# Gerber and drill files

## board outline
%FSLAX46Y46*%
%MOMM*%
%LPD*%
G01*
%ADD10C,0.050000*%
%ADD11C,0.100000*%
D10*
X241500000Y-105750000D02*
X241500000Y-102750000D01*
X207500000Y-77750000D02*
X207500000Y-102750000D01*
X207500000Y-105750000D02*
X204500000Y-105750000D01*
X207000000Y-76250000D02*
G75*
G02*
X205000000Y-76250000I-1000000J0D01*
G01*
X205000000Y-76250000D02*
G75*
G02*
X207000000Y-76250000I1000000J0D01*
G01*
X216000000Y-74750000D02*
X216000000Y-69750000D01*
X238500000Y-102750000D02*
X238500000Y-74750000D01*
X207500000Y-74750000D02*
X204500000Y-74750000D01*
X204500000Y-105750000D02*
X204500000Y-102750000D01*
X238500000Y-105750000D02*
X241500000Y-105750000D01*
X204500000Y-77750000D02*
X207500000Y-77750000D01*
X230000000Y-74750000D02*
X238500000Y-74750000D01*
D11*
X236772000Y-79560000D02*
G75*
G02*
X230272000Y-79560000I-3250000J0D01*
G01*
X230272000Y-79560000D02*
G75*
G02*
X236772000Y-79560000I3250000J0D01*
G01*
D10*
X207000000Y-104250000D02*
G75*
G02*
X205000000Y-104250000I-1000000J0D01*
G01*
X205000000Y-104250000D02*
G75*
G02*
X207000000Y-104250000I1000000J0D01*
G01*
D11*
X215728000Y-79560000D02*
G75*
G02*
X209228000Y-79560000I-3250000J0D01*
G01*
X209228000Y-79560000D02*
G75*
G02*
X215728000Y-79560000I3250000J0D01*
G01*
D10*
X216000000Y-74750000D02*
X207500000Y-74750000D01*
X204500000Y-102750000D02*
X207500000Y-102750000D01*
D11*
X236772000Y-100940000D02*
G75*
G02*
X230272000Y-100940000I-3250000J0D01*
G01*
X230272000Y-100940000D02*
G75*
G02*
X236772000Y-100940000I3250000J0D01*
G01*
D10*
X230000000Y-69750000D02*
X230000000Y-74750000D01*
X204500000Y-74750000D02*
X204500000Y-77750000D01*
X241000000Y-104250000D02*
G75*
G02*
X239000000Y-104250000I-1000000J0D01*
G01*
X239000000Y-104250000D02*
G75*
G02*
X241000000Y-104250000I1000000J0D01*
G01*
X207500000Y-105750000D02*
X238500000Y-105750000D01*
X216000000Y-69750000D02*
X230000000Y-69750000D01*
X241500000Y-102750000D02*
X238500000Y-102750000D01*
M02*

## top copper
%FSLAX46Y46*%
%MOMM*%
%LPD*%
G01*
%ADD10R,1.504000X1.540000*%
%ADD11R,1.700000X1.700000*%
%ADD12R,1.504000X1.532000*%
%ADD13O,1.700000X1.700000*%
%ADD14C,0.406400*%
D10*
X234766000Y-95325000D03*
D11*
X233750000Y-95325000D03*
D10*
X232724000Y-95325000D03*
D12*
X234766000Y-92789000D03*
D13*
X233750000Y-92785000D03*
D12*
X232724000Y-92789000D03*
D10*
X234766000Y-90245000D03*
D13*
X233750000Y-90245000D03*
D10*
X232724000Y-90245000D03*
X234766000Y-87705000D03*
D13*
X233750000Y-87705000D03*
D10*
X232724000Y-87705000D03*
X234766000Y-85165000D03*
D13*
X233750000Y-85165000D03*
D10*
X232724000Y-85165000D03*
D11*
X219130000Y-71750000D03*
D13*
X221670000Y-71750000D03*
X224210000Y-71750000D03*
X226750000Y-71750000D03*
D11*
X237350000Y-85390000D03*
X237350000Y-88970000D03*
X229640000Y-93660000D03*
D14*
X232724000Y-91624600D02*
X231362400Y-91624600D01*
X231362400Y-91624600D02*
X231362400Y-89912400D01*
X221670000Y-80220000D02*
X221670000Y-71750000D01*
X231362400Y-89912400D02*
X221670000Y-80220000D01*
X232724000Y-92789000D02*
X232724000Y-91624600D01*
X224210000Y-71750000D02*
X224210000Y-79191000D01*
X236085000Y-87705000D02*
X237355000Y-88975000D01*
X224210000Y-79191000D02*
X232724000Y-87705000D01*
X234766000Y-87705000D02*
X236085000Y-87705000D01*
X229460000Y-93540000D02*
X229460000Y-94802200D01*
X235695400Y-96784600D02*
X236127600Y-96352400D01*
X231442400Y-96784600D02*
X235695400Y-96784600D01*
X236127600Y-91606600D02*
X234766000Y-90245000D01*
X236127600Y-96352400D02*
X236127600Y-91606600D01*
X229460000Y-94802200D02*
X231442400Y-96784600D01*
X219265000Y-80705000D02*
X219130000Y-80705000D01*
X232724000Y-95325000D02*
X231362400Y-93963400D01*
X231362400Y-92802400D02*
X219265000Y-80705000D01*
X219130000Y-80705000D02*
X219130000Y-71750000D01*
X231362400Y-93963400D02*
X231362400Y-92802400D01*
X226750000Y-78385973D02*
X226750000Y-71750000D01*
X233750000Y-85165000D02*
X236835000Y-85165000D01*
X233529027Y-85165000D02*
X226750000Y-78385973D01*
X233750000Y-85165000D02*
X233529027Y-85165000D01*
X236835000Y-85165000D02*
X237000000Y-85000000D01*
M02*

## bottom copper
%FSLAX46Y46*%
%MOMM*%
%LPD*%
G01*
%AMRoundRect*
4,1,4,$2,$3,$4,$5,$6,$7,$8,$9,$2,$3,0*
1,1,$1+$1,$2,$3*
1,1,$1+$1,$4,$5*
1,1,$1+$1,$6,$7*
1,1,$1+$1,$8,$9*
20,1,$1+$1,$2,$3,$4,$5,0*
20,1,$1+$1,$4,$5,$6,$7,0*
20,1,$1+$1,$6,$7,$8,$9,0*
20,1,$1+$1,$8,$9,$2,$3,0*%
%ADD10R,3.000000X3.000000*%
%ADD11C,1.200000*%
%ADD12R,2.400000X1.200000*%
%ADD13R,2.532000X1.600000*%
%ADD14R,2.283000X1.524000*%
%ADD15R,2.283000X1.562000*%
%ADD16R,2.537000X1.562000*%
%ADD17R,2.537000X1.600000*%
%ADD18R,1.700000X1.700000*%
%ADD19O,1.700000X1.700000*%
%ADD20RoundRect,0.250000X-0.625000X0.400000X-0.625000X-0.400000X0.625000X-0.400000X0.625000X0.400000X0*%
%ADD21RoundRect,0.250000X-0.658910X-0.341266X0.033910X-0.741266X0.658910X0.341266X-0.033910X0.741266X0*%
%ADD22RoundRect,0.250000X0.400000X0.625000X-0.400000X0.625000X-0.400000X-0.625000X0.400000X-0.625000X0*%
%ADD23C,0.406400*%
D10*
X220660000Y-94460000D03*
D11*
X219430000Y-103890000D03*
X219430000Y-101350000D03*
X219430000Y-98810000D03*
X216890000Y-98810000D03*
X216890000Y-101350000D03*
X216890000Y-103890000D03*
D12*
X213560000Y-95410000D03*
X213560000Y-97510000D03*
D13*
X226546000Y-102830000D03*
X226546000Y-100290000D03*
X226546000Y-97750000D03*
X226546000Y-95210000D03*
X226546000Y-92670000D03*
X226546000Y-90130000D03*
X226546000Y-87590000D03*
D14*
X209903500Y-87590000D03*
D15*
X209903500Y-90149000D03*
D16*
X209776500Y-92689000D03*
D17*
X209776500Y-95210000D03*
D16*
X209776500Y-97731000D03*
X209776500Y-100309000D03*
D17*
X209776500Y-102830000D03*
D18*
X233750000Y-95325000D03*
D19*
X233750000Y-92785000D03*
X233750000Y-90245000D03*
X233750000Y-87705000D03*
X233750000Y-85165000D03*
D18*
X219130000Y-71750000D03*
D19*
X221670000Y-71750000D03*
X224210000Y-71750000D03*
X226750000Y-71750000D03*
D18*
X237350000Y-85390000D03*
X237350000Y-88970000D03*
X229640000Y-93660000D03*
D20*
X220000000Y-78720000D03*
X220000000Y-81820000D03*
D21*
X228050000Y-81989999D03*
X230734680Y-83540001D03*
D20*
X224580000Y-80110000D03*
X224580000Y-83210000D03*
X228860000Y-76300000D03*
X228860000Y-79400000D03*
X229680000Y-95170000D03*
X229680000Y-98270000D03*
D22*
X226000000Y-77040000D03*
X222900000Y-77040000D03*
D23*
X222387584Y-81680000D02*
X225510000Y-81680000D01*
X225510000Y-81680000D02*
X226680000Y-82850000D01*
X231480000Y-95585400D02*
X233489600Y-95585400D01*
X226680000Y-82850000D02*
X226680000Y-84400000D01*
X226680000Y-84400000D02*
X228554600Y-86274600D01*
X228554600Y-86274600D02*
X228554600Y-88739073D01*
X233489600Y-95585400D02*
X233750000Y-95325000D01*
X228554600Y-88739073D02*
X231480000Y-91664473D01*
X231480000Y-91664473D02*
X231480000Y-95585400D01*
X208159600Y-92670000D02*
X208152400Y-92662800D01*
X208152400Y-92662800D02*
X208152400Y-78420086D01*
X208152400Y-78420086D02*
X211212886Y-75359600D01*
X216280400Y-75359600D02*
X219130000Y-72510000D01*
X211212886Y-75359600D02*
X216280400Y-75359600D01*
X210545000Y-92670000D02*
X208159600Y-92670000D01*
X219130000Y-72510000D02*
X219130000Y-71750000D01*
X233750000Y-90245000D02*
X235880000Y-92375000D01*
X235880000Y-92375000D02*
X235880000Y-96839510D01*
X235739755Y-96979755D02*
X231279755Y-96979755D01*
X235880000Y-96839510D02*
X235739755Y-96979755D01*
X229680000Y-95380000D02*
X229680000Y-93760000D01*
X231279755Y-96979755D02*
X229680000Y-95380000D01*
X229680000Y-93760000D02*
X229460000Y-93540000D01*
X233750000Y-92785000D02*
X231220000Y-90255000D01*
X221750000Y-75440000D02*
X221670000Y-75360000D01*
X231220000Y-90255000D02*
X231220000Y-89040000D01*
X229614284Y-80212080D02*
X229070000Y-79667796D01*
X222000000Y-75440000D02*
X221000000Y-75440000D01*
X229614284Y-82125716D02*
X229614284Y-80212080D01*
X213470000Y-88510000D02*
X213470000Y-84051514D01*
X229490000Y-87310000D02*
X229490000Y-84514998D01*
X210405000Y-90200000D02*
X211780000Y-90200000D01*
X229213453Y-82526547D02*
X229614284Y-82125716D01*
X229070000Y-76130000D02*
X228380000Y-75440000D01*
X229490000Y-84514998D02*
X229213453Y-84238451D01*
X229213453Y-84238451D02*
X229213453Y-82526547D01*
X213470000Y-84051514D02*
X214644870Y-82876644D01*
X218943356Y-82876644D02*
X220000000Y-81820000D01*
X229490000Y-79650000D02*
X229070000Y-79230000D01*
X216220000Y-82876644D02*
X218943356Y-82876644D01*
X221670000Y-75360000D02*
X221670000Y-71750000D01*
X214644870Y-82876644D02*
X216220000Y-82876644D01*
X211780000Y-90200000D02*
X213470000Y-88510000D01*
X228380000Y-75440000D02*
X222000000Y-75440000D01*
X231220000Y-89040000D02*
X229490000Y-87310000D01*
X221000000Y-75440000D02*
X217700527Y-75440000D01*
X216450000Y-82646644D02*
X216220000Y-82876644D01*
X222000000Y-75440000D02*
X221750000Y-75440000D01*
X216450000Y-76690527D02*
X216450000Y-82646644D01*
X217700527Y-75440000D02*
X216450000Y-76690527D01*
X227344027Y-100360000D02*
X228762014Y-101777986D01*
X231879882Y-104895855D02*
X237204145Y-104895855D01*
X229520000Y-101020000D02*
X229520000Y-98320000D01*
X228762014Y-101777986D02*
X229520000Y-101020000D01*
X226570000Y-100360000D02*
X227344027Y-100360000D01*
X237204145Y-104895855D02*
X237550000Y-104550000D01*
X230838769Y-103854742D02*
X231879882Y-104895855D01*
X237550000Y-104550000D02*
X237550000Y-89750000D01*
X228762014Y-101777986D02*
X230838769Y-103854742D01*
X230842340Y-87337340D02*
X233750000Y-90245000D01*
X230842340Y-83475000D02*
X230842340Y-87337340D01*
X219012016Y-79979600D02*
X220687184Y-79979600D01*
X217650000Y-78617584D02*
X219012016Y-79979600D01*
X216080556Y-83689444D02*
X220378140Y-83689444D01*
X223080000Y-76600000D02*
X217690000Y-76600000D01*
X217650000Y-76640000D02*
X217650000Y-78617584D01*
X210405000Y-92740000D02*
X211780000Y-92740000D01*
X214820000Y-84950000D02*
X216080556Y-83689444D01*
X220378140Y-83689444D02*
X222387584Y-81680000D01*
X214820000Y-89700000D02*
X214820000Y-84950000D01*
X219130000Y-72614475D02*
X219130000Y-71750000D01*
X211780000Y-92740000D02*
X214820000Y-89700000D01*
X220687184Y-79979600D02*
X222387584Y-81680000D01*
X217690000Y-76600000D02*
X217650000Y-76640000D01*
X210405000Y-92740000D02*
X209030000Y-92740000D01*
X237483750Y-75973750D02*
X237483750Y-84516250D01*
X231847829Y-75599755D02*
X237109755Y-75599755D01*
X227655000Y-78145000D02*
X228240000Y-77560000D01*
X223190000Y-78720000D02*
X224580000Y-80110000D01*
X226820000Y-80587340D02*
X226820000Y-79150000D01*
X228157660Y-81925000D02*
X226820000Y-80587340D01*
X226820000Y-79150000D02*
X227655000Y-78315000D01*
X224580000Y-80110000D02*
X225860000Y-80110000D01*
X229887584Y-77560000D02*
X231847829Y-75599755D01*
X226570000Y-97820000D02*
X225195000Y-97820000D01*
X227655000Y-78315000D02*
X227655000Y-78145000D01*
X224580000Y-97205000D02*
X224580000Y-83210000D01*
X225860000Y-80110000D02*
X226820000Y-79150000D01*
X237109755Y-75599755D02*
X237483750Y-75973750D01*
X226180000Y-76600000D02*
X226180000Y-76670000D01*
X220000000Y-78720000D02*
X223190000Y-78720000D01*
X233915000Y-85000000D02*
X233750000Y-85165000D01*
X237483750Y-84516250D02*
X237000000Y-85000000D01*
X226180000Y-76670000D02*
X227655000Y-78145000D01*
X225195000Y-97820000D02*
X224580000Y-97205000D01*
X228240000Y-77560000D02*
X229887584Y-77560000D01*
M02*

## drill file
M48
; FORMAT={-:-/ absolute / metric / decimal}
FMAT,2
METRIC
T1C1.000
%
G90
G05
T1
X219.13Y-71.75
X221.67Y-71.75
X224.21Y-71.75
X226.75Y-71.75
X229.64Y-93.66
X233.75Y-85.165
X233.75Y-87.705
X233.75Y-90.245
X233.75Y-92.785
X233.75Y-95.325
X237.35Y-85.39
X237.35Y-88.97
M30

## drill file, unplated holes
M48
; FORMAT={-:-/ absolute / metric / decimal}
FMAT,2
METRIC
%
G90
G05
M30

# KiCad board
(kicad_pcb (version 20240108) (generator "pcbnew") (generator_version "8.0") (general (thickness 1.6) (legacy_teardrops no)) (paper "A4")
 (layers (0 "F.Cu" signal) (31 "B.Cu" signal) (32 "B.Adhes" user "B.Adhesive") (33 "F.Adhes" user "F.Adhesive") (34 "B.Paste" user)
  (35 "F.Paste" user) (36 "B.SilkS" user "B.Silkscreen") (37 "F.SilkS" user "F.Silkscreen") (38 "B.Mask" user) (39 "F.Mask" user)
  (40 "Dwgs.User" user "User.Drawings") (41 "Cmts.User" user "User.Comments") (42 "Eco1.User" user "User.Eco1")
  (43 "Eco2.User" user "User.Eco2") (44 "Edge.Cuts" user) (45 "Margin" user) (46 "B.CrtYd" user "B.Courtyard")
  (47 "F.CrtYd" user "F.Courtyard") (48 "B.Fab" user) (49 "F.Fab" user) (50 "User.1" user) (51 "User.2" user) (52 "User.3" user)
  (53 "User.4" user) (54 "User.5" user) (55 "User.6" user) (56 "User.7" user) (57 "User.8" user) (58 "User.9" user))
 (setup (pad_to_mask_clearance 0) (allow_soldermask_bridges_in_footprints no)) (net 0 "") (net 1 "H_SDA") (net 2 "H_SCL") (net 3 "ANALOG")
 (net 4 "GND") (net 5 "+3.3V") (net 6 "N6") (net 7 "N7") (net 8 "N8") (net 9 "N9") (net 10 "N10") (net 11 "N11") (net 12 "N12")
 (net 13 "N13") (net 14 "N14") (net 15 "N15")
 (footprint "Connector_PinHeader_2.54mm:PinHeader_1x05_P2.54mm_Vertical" (layer "F.Cu") (at 233.75 95.325 180)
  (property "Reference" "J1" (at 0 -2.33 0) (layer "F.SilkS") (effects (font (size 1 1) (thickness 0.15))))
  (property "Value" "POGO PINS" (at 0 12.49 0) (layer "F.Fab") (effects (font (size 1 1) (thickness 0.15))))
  (pad "1" smd rect (at -1.016 0 180) (size 1.504 1.54) (layers "F.Cu" "F.Paste" "F.Mask") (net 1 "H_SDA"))
  (pad "1" thru_hole rect (at 0 0 180) (size 1.7 1.7) (drill 1) (layers "*.Cu" "*.Mask") (remove_unused_layers no) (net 1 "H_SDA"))
  (pad "1" smd rect (at 1.026 0 180) (size 1.504 1.54) (layers "F.Cu" "F.Paste" "F.Mask") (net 1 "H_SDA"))
  (pad "2" smd rect (at -1.016 2.536 180) (size 1.504 1.532) (layers "F.Cu" "F.Paste" "F.Mask") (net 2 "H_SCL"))
  (pad "2" thru_hole oval (at 0 2.54 180) (size 1.7 1.7) (drill 1) (layers "*.Cu" "*.Mask") (remove_unused_layers no) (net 2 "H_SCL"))
  (pad "2" smd rect (at 1.026 2.536 180) (size 1.504 1.532) (layers "F.Cu" "F.Paste" "F.Mask") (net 2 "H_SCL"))
  (pad "3" smd rect (at -1.016 5.08 180) (size 1.504 1.54) (layers "F.Cu" "F.Paste" "F.Mask") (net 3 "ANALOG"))
  (pad "3" thru_hole oval (at 0 5.08 180) (size 1.7 1.7) (drill 1) (layers "*.Cu" "*.Mask") (remove_unused_layers no) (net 3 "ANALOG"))
  (pad "3" smd rect (at 1.026 5.08 180) (size 1.504 1.54) (layers "F.Cu" "F.Paste" "F.Mask") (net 3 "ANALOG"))
  (pad "4" smd rect (at -1.016 7.62 180) (size 1.504 1.54) (layers "F.Cu" "F.Paste" "F.Mask") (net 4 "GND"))
  (pad "4" thru_hole oval (at 0 7.62 180) (size 1.7 1.7) (drill 1) (layers "*.Cu" "*.Mask") (remove_unused_layers no) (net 4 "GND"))
  (pad "4" smd rect (at 1.026 7.62 180) (size 1.504 1.54) (layers "F.Cu" "F.Paste" "F.Mask") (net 4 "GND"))
  (pad "5" smd rect (at -1.016 10.16 180) (size 1.504 1.54) (layers "F.Cu" "F.Paste" "F.Mask") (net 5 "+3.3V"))
  (pad "5" thru_hole oval (at 0 10.16 180) (size 1.7 1.7) (drill 1) (layers "*.Cu" "*.Mask") (remove_unused_layers no) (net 5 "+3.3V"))
  (pad "5" smd rect (at 1.026 10.16 180) (size 1.504 1.54) (layers "F.Cu" "F.Paste" "F.Mask") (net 5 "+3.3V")))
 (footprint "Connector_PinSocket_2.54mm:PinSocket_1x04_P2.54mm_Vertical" (layer "F.Cu") (at 219.13 71.75 90)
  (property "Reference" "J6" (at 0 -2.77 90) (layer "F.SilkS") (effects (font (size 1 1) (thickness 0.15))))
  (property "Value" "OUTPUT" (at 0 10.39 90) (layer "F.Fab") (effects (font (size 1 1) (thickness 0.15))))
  (pad "1" thru_hole rect (at 0 0 90) (size 1.7 1.7) (drill 1) (layers "*.Cu" "*.Mask") (remove_unused_layers no) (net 1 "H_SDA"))
  (pad "2" thru_hole oval (at 0 2.54 90) (size 1.7 1.7) (drill 1) (layers "*.Cu" "*.Mask") (remove_unused_layers no) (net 2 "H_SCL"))
  (pad "3" thru_hole oval (at 0 5.08 90) (size 1.7 1.7) (drill 1) (layers "*.Cu" "*.Mask") (remove_unused_layers no) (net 4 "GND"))
  (pad "4" thru_hole oval (at 0 7.62 90) (size 1.7 1.7) (drill 1) (layers "*.Cu" "*.Mask") (remove_unused_layers no) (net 5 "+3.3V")))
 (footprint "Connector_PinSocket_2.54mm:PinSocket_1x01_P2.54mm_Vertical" (layer "F.Cu") (at 237.35 85.39)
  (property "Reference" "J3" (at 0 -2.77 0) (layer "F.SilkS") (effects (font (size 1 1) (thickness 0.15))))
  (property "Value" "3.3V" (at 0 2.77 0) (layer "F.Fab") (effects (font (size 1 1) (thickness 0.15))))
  (pad "1" thru_hole rect (at 0 0) (size 1.7 1.7) (drill 1) (layers "*.Cu" "*.Mask") (remove_unused_layers no) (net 5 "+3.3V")))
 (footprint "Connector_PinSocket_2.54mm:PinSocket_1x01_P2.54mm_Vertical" (layer "F.Cu") (at 237.35 88.97)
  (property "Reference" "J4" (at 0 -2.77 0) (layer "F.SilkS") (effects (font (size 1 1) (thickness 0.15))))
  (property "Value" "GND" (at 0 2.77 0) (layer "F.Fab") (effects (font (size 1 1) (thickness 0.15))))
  (pad "1" thru_hole rect (at 0 0) (size 1.7 1.7) (drill 1) (layers "*.Cu" "*.Mask") (remove_unused_layers no) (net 4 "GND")))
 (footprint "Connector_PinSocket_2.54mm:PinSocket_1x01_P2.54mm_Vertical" (layer "F.Cu") (at 229.64 93.66)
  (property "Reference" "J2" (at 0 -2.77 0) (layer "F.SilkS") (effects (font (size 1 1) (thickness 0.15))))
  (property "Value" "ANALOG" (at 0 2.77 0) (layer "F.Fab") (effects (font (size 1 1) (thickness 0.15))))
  (pad "1" thru_hole rect (at 0 0) (size 1.7 1.7) (drill 1) (layers "*.Cu" "*.Mask") (remove_unused_layers no) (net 3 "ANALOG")))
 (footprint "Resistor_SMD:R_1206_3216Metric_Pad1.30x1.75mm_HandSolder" (layer "B.Cu") (at 220 80.27 -90)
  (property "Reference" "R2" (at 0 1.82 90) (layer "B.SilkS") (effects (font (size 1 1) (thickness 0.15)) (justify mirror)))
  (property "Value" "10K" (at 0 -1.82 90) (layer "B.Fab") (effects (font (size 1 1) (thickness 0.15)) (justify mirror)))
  (pad "1" smd roundrect (at -1.55 0 270) (size 1.3 1.75) (layers "B.Cu" "B.Paste" "B.Mask") (roundrect_rratio 0.192308) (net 5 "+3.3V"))
  (pad "2" smd roundrect (at 1.55 0 270) (size 1.3 1.75) (layers "B.Cu" "B.Paste" "B.Mask") (roundrect_rratio 0.192308) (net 2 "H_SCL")))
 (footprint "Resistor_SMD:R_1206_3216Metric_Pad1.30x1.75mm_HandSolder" (layer "B.Cu") (at 229.39234 82.765 -30)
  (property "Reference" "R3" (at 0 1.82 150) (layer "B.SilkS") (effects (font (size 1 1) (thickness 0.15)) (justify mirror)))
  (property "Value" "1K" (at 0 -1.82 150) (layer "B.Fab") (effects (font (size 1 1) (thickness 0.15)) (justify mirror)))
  (pad "1" smd roundrect (at -1.550001 -0.000001 330) (size 1.3 1.75) (layers "B.Cu" "B.Paste" "B.Mask") (roundrect_rratio 0.192308)
   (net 5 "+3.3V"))
  (pad "2" smd roundrect (at 1.550001 0.000001 330) (size 1.3 1.75) (layers "B.Cu" "B.Paste" "B.Mask") (roundrect_rratio 0.192308)
   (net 3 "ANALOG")))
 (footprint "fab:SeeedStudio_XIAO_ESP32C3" (layer "B.Cu") (at 218.16 95.21)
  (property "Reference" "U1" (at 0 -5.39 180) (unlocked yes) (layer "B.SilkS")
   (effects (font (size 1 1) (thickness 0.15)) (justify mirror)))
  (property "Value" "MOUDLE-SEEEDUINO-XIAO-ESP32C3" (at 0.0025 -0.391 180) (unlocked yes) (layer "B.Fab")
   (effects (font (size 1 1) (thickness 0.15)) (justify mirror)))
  (pad "1" smd rect (at -7.615 7.62) (size 2.537 1.6) (drill (offset -0.7685 0)) (layers "B.Cu" "B.Paste" "B.Mask") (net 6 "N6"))
  (pad "2" smd rect (at -7.615 5.08) (size 2.537 1.562) (drill (offset -0.7685 0.019)) (layers "B.Cu" "B.Paste" "B.Mask") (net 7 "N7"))
  (pad "3" smd rect (at -7.615 2.54) (size 2.537 1.562) (drill (offset -0.7685 -0.019)) (layers "B.Cu" "B.Paste" "B.Mask") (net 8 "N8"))
  (pad "4" smd rect (at -7.615 0) (size 2.537 1.6) (drill (offset -0.7685 0)) (layers "B.Cu" "B.Paste" "B.Mask") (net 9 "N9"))
  (pad "5" smd rect (at -7.615 -2.54) (size 2.537 1.562) (drill (offset -0.7685 0.019)) (layers "B.Cu" "B.Paste" "B.Mask") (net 1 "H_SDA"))
  (pad "6" smd rect (at -7.615 -5.08) (size 2.283 1.562) (drill (offset -0.6415 0.019)) (layers "B.Cu" "B.Paste" "B.Mask") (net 2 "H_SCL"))
  (pad "7" smd rect (at -7.615 -7.62) (size 2.283 1.524) (drill (offset -0.6415 0)) (layers "B.Cu" "B.Paste" "B.Mask") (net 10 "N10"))
  (pad "8" smd rect (at 7.62 -7.62) (size 2.532 1.6) (drill (offset 0.766 0)) (layers "B.Cu" "B.Paste" "B.Mask") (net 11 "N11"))
  (pad "9" smd rect (at 7.62 -5.08) (size 2.532 1.6) (drill (offset 0.766 0)) (layers "B.Cu" "B.Paste" "B.Mask") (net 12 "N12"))
  (pad "10" smd rect (at 7.62 -2.54) (size 2.532 1.6) (drill (offset 0.766 0)) (layers "B.Cu" "B.Paste" "B.Mask") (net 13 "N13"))
  (pad "11" smd rect (at 7.62 0) (size 2.532 1.6) (drill (offset 0.766 0)) (layers "B.Cu" "B.Paste" "B.Mask") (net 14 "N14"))
  (pad "12" smd rect (at 7.62 2.54) (size 2.532 1.6) (drill (offset 0.766 0)) (layers "B.Cu" "B.Paste" "B.Mask") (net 5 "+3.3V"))
  (pad "13" smd rect (at 7.62 5.08) (size 2.532 1.6) (drill (offset 0.766 0)) (layers "B.Cu" "B.Paste" "B.Mask") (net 4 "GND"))
  (pad "14" smd rect (at 7.62 7.62) (size 2.532 1.6) (drill (offset 0.766 0)) (layers "B.Cu" "B.Paste" "B.Mask") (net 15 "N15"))
  (pad "15" smd rect (at -4.6 2.3) (size 2.4 1.2) (layers "B.Cu" "B.Paste" "B.Mask"))
  (pad "16" smd rect (at -4.6 0.2) (size 2.4 1.2) (layers "B.Cu" "B.Paste" "B.Mask"))
  (pad "17" smd circle (at -1.27 8.68) (size 1.2 1.2) (layers "B.Cu" "B.Paste" "B.Mask"))
  (pad "18" smd circle (at -1.27 6.14) (size 1.2 1.2) (layers "B.Cu" "B.Paste" "B.Mask"))
  (pad "19" smd circle (at -1.27 3.6) (size 1.2 1.2) (layers "B.Cu" "B.Paste" "B.Mask"))
  (pad "20" smd circle (at 1.27 3.6) (size 1.2 1.2) (layers "B.Cu" "B.Paste" "B.Mask"))
  (pad "21" smd circle (at 1.27 6.14) (size 1.2 1.2) (layers "B.Cu" "B.Paste" "B.Mask"))
  (pad "22" smd circle (at 1.27 8.68) (size 1.2 1.2) (layers "B.Cu" "B.Paste" "B.Mask"))
  (pad "23" smd rect (at 2.5 -0.75) (size 3 3) (layers "B.Cu" "B.Paste" "B.Mask")))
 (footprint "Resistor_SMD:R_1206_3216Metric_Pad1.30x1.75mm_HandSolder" (layer "B.Cu") (at 224.58 81.66 -90)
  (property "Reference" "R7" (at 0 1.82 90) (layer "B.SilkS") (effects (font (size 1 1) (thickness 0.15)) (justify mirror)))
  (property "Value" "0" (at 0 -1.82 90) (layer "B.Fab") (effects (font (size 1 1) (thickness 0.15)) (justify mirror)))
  (pad "1" smd roundrect (at -1.55 0 270) (size 1.3 1.75) (layers "B.Cu" "B.Paste" "B.Mask") (roundrect_rratio 0.192308) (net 5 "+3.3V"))
  (pad "2" smd roundrect (at 1.55 0 270) (size 1.3 1.75) (layers "B.Cu" "B.Paste" "B.Mask") (roundrect_rratio 0.192308) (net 5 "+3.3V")))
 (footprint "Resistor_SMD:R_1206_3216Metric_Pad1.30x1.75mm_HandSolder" (layer "B.Cu") (at 228.86 77.85 -90)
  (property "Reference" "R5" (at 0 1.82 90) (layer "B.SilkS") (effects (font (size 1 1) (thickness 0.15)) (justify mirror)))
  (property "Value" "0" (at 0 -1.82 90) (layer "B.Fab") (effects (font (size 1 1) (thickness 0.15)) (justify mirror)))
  (pad "1" smd roundrect (at -1.55 0 270) (size 1.3 1.75) (layers "B.Cu" "B.Paste" "B.Mask") (roundrect_rratio 0.192308) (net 2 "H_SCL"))
  (pad "2" smd roundrect (at 1.55 0 270) (size 1.3 1.75) (layers "B.Cu" "B.Paste" "B.Mask") (roundrect_rratio 0.192308) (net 2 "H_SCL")))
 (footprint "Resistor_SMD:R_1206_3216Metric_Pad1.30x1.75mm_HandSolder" (layer "B.Cu") (at 229.68 96.72 -90)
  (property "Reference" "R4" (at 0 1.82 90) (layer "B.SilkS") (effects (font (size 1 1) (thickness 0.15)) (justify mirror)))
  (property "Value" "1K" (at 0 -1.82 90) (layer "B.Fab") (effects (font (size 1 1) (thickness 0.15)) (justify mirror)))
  (pad "1" smd roundrect (at -1.55 0 270) (size 1.3 1.75) (layers "B.Cu" "B.Paste" "B.Mask") (roundrect_rratio 0.192308) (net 3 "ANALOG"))
  (pad "2" smd roundrect (at 1.55 0 270) (size 1.3 1.75) (layers "B.Cu" "B.Paste" "B.Mask") (roundrect_rratio 0.192308) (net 4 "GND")))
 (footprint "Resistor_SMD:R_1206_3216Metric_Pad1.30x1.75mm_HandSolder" (layer "B.Cu") (at 224.45 77.04 180)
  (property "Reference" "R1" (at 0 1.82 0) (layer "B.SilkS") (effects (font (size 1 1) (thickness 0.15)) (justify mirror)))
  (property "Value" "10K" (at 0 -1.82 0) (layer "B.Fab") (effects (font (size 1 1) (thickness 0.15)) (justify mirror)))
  (pad "1" smd roundrect (at -1.55 0 180) (size 1.3 1.75) (layers "B.Cu" "B.Paste" "B.Mask") (roundrect_rratio 0.192308) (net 5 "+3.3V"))
  (pad "2" smd roundrect (at 1.55 0 180) (size 1.3 1.75) (layers "B.Cu" "B.Paste" "B.Mask") (roundrect_rratio 0.192308) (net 1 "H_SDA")))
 (gr_line (start 241.5 105.75) (end 241.5 102.75) (stroke (width 0.05) (type default)) (layer "Edge.Cuts"))
 (gr_line (start 207.5 77.75) (end 207.5 102.75) (stroke (width 0.05) (type default)) (layer "Edge.Cuts"))
 (gr_line (start 207.5 105.75) (end 204.5 105.75) (stroke (width 0.05) (type default)) (layer "Edge.Cuts"))
 (gr_circle (center 206 76.25) (end 206 77.25) (stroke (width 0.05) (type default)) (fill none) (layer "Edge.Cuts"))
 (gr_line (start 216 74.75) (end 216 69.75) (stroke (width 0.05) (type default)) (layer "Edge.Cuts"))
 (gr_line (start 238.5 102.75) (end 238.5 74.75) (stroke (width 0.05) (type default)) (layer "Edge.Cuts"))
 (gr_line (start 207.5 74.75) (end 204.5 74.75) (stroke (width 0.05) (type default)) (layer "Edge.Cuts"))
 (gr_line (start 204.5 105.75) (end 204.5 102.75) (stroke (width 0.05) (type default)) (layer "Edge.Cuts"))
 (gr_line (start 238.5 105.75) (end 241.5 105.75) (stroke (width 0.05) (type default)) (layer "Edge.Cuts"))
 (gr_line (start 204.5 77.75) (end 207.5 77.75) (stroke (width 0.05) (type default)) (layer "Edge.Cuts"))
 (gr_line (start 230 74.75) (end 238.5 74.75) (stroke (width 0.05) (type default)) (layer "Edge.Cuts"))
 (gr_circle (center 233.522 79.56) (end 230.272 79.56) (stroke (width 0.1) (type default)) (fill none) (layer "Edge.Cuts"))
 (gr_circle (center 206 104.25) (end 206 105.25) (stroke (width 0.05) (type default)) (fill none) (layer "Edge.Cuts"))
 (gr_circle (center 212.478 79.56) (end 209.228 79.56) (stroke (width 0.1) (type default)) (fill none) (layer "Edge.Cuts"))
 (gr_line (start 216 74.75) (end 207.5 74.75) (stroke (width 0.05) (type default)) (layer "Edge.Cuts"))
 (gr_line (start 204.5 102.75) (end 207.5 102.75) (stroke (width 0.05) (type default)) (layer "Edge.Cuts"))
 (gr_circle (center 233.522 100.94) (end 230.272 100.94) (stroke (width 0.1) (type default)) (fill none) (layer "Edge.Cuts"))
 (gr_line (start 230 69.75) (end 230 74.75) (stroke (width 0.05) (type default)) (layer "Edge.Cuts"))
 (gr_line (start 204.5 74.75) (end 204.5 77.75) (stroke (width 0.05) (type default)) (layer "Edge.Cuts"))
 (gr_circle (center 240 104.25) (end 240 105.25) (stroke (width 0.05) (type default)) (fill none) (layer "Edge.Cuts"))
 (gr_line (start 207.5 105.75) (end 238.5 105.75) (stroke (width 0.05) (type default)) (layer "Edge.Cuts"))
 (gr_line (start 216 69.75) (end 230 69.75) (stroke (width 0.05) (type default)) (layer "Edge.Cuts"))
 (gr_line (start 241.5 102.75) (end 238.5 102.75) (stroke (width 0.05) (type default)) (layer "Edge.Cuts"))
 (segment (start 232.724 91.6246) (end 231.3624 91.6246) (width 0.4064) (layer "F.Cu") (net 2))
 (segment (start 231.3624 91.6246) (end 231.3624 89.9124) (width 0.4064) (layer "F.Cu") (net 2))
 (segment (start 221.67 80.22) (end 221.67 71.75) (width 0.4064) (layer "F.Cu") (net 2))
 (segment (start 231.3624 89.9124) (end 221.67 80.22) (width 0.4064) (layer "F.Cu") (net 2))
 (segment (start 232.724 92.789) (end 232.724 91.6246) (width 0.4064) (layer "F.Cu") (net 2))
 (segment (start 233.75 92.785) (end 231.22 90.255) (width 0.4064) (layer "B.Cu") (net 2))
 (segment (start 221.75 75.44) (end 221.67 75.36) (width 0.4064) (layer "B.Cu") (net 2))
 (segment (start 231.22 90.255) (end 231.22 89.04) (width 0.4064) (layer "B.Cu") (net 2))
 (segment (start 229.614284 80.21208) (end 229.07 79.667796) (width 0.4064) (layer "B.Cu") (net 2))
 (segment (start 222 75.44) (end 221 75.44) (width 0.4064) (layer "B.Cu") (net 2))
 (segment (start 229.614284 82.125716) (end 229.614284 80.21208) (width 0.4064) (layer "B.Cu") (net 2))
 (segment (start 213.47 88.51) (end 213.47 84.051514) (width 0.4064) (layer "B.Cu") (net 2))
 (segment (start 229.49 87.31) (end 229.49 84.514998) (width 0.4064) (layer "B.Cu") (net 2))
 (segment (start 210.405 90.2) (end 211.78 90.2) (width 0.4064) (layer "B.Cu") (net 2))
 (segment (start 229.213453 82.526547) (end 229.614284 82.125716) (width 0.4064) (layer "B.Cu") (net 2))
 (segment (start 229.07 76.13) (end 228.38 75.44) (width 0.4064) (layer "B.Cu") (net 2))
 (segment (start 229.49 84.514998) (end 229.213453 84.238451) (width 0.4064) (layer "B.Cu") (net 2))
 (segment (start 229.213453 84.238451) (end 229.213453 82.526547) (width 0.4064) (layer "B.Cu") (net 2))
 (segment (start 213.47 84.051514) (end 214.64487 82.876644) (width 0.4064) (layer "B.Cu") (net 2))
 (segment (start 218.943356 82.876644) (end 220 81.82) (width 0.4064) (layer "B.Cu") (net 2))
 (segment (start 229.49 79.65) (end 229.07 79.23) (width 0.4064) (layer "B.Cu") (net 2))
 (segment (start 216.22 82.876644) (end 218.943356 82.876644) (width 0.4064) (layer "B.Cu") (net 2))
 (segment (start 221.67 75.36) (end 221.67 71.75) (width 0.4064) (layer "B.Cu") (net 2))
 (segment (start 214.64487 82.876644) (end 216.22 82.876644) (width 0.4064) (layer "B.Cu") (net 2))
 (segment (start 211.78 90.2) (end 213.47 88.51) (width 0.4064) (layer "B.Cu") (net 2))
 (segment (start 228.38 75.44) (end 222 75.44) (width 0.4064) (layer "B.Cu") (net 2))
 (segment (start 231.22 89.04) (end 229.49 87.31) (width 0.4064) (layer "B.Cu") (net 2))
 (segment (start 221 75.44) (end 217.700527 75.44) (width 0.4064) (layer "B.Cu") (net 2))
 (segment (start 216.45 82.646644) (end 216.22 82.876644) (width 0.4064) (layer "B.Cu") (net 2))
 (segment (start 222 75.44) (end 221.75 75.44) (width 0.4064) (layer "B.Cu") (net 2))
 (segment (start 216.45 76.690527) (end 216.45 82.646644) (width 0.4064) (layer "B.Cu") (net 2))
 (segment (start 217.700527 75.44) (end 216.45 76.690527) (width 0.4064) (layer "B.Cu") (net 2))
 (segment (start 224.21 71.75) (end 224.21 79.191) (width 0.4064) (layer "F.Cu") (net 4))
 (segment (start 236.085 87.705) (end 237.355 88.975) (width 0.4064) (layer "F.Cu") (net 4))
 (segment (start 224.21 79.191) (end 232.724 87.705) (width 0.4064) (layer "F.Cu") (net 4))
 (segment (start 234.766 87.705) (end 236.085 87.705) (width 0.4064) (layer "F.Cu") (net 4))
 (segment (start 227.344027 100.36) (end 228.762014 101.777986) (width 0.4064) (layer "B.Cu") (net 4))
 (segment (start 231.879882 104.895855) (end 237.204145 104.895855) (width 0.4064) (layer "B.Cu") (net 4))
 (segment (start 229.52 101.02) (end 229.52 98.32) (width 0.4064) (layer "B.Cu") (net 4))
 (segment (start 228.762014 101.777986) (end 229.52 101.02) (width 0.4064) (layer "B.Cu") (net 4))
 (segment (start 226.57 100.36) (end 227.344027 100.36) (width 0.4064) (layer "B.Cu") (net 4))
 (segment (start 237.204145 104.895855) (end 237.55 104.55) (width 0.4064) (layer "B.Cu") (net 4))
 (segment (start 230.838769 103.854742) (end 231.879882 104.895855) (width 0.4064) (layer "B.Cu") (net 4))
 (segment (start 237.55 104.55) (end 237.55 89.75) (width 0.4064) (layer "B.Cu") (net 4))
 (segment (start 228.762014 101.777986) (end 230.838769 103.854742) (width 0.4064) (layer "B.Cu") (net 4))
 (segment (start 229.46 93.54) (end 229.46 94.8022) (width 0.4064) (layer "F.Cu") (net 3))
 (segment (start 235.6954 96.7846) (end 236.1276 96.3524) (width 0.4064) (layer "F.Cu") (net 3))
 (segment (start 231.4424 96.7846) (end 235.6954 96.7846) (width 0.4064) (layer "F.Cu") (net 3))
 (segment (start 236.1276 91.6066) (end 234.766 90.245) (width 0.4064) (layer "F.Cu") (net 3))
 (segment (start 236.1276 96.3524) (end 236.1276 91.6066) (width 0.4064) (layer "F.Cu") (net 3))
 (segment (start 229.46 94.8022) (end 231.4424 96.7846) (width 0.4064) (layer "F.Cu") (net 3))
 (segment (start 235.88 92.375) (end 235.88 96.83951) (width 0.4064) (layer "B.Cu") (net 3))
 (segment (start 233.75 90.245) (end 235.88 92.375) (width 0.4064) (layer "B.Cu") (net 3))
 (segment (start 235.88 96.83951) (end 235.739755 96.979755) (width 0.4064) (layer "B.Cu") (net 3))
 (segment (start 229.68 95.38) (end 229.68 93.76) (width 0.4064) (layer "B.Cu") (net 3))
 (segment (start 235.739755 96.979755) (end 231.279755 96.979755) (width 0.4064) (layer "B.Cu") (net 3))
 (segment (start 229.68 93.76) (end 229.46 93.54) (width 0.4064) (layer "B.Cu") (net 3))
 (segment (start 231.279755 96.979755) (end 229.68 95.38) (width 0.4064) (layer "B.Cu") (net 3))
 (segment (start 230.84234 87.33734) (end 233.75 90.245) (width 0.4064) (layer "B.Cu") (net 3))
 (segment (start 230.84234 83.475) (end 230.84234 87.33734) (width 0.4064) (layer "B.Cu") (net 3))
 (segment (start 219.265 80.705) (end 219.13 80.705) (width 0.4064) (layer "F.Cu") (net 1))
 (segment (start 232.724 95.325) (end 231.3624 93.9634) (width 0.4064) (layer "F.Cu") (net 1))
 (segment (start 231.3624 92.8024) (end 219.265 80.705) (width 0.4064) (layer "F.Cu") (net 1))
 (segment (start 219.13 80.705) (end 219.13 71.75) (width 0.4064) (layer "F.Cu") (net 1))
 (segment (start 231.3624 93.9634) (end 231.3624 92.8024) (width 0.4064) (layer "F.Cu") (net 1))
 (segment (start 219.012016 79.9796) (end 220.687184 79.9796) (width 0.4064) (layer "B.Cu") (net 1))
 (segment (start 217.65 78.617584) (end 219.012016 79.9796) (width 0.4064) (layer "B.Cu") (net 1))
 (segment (start 231.48 91.664473) (end 231.48 95.5854) (width 0.4064) (layer "B.Cu") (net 1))
 (segment (start 216.080556 83.689444) (end 220.37814 83.689444) (width 0.4064) (layer "B.Cu") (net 1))
 (segment (start 223.08 76.6) (end 217.69 76.6) (width 0.4064) (layer "B.Cu") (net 1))
 (segment (start 217.65 76.64) (end 217.65 78.617584) (width 0.4064) (layer "B.Cu") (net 1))
 (segment (start 233.4896 95.5854) (end 233.75 95.325) (width 0.4064) (layer "B.Cu") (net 1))
 (segment (start 226.68 84.4) (end 228.5546 86.2746) (width 0.4064) (layer "B.Cu") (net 1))
 (segment (start 210.405 92.74) (end 211.78 92.74) (width 0.4064) (layer "B.Cu") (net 1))
 (segment (start 226.68 82.85) (end 226.68 84.4) (width 0.4064) (layer "B.Cu") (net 1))
 (segment (start 208.1524 78.420086) (end 211.212886 75.3596) (width 0.4064) (layer "B.Cu") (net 1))
 (segment (start 214.82 84.95) (end 216.080556 83.689444) (width 0.4064) (layer "B.Cu") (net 1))
 (segment (start 211.212886 75.3596) (end 216.2804 75.3596) (width 0.4064) (layer "B.Cu") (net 1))
 (segment (start 231.48 95.5854) (end 233.4896 95.5854) (width 0.4064) (layer "B.Cu") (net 1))
 (segment (start 219.13 72.51) (end 219.13 71.75) (width 0.4064) (layer "B.Cu") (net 1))
 (segment (start 208.1524 92.6628) (end 208.1524 78.420086) (width 0.4064) (layer "B.Cu") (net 1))
 (segment (start 220.37814 83.689444) (end 222.387584 81.68) (width 0.4064) (layer "B.Cu") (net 1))
 (segment (start 208.1596 92.67) (end 208.1524 92.6628) (width 0.4064) (layer "B.Cu") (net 1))
 (segment (start 214.82 89.7) (end 214.82 84.95) (width 0.4064) (layer "B.Cu") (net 1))
 (segment (start 222.387584 81.68) (end 225.51 81.68) (width 0.4064) (layer "B.Cu") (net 1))
 (segment (start 219.13 72.614475) (end 219.13 71.75) (width 0.4064) (layer "B.Cu") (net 1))
 (segment (start 211.78 92.74) (end 214.82 89.7) (width 0.4064) (layer "B.Cu") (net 1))
 (segment (start 228.5546 88.739073) (end 231.48 91.664473) (width 0.4064) (layer "B.Cu") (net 1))
 (segment (start 220.687184 79.9796) (end 222.387584 81.68) (width 0.4064) (layer "B.Cu") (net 1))
 (segment (start 217.69 76.6) (end 217.65 76.64) (width 0.4064) (layer "B.Cu") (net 1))
 (segment (start 216.2804 75.3596) (end 219.13 72.51) (width 0.4064) (layer "B.Cu") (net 1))
 (segment (start 225.51 81.68) (end 226.68 82.85) (width 0.4064) (layer "B.Cu") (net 1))
 (segment (start 210.545 92.67) (end 208.1596 92.67) (width 0.4064) (layer "B.Cu") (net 1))
 (segment (start 210.405 92.74) (end 209.03 92.74) (width 0.4064) (layer "B.Cu") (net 1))
 (segment (start 228.5546 86.2746) (end 228.5546 88.739073) (width 0.4064) (layer "B.Cu") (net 1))
 (segment (start 226.75 78.385973) (end 226.75 71.75) (width 0.4064) (layer "F.Cu") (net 5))
 (segment (start 233.75 85.165) (end 236.835 85.165) (width 0.4064) (layer "F.Cu") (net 5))
 (segment (start 233.529027 85.165) (end 226.75 78.385973) (width 0.4064) (layer "F.Cu") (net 5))
 (segment (start 233.75 85.165) (end 233.529027 85.165) (width 0.4064) (layer "F.Cu") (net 5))
 (segment (start 236.835 85.165) (end 237 85) (width 0.4064) (layer "F.Cu") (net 5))
 (segment (start 237.48375 75.97375) (end 237.48375 84.51625) (width 0.4064) (layer "B.Cu") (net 5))
 (segment (start 231.847829 75.599755) (end 237.109755 75.599755) (width 0.4064) (layer "B.Cu") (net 5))
 (segment (start 227.655 78.145) (end 228.24 77.56) (width 0.4064) (layer "B.Cu") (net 5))
 (segment (start 223.19 78.72) (end 224.58 80.11) (width 0.4064) (layer "B.Cu") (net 5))
 (segment (start 226.82 80.58734) (end 226.82 79.15) (width 0.4064) (layer "B.Cu") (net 5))
 (segment (start 228.15766 81.925) (end 226.82 80.58734) (width 0.4064) (layer "B.Cu") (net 5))
 (segment (start 226.82 79.15) (end 227.655 78.315) (width 0.4064) (layer "B.Cu") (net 5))
 (segment (start 224.58 80.11) (end 225.86 80.11) (width 0.4064) (layer "B.Cu") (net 5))
 (segment (start 229.887584 77.56) (end 231.847829 75.599755) (width 0.4064) (layer "B.Cu") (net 5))
 (segment (start 226.57 97.82) (end 225.195 97.82) (width 0.4064) (layer "B.Cu") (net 5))
 (segment (start 227.655 78.315) (end 227.655 78.145) (width 0.4064) (layer "B.Cu") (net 5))
 (segment (start 224.58 97.205) (end 224.58 83.21) (width 0.4064) (layer "B.Cu") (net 5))
 (segment (start 225.86 80.11) (end 226.82 79.15) (width 0.4064) (layer "B.Cu") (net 5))
 (segment (start 237.109755 75.599755) (end 237.48375 75.97375) (width 0.4064) (layer "B.Cu") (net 5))
 (segment (start 226.18 76.6) (end 226.18 76.67) (width 0.4064) (layer "B.Cu") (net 5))
 (segment (start 220 78.72) (end 223.19 78.72) (width 0.4064) (layer "B.Cu") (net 5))
 (segment (start 233.915 85) (end 233.75 85.165) (width 0.4064) (layer "B.Cu") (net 5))
 (segment (start 237.48375 84.51625) (end 237 85) (width 0.4064) (layer "B.Cu") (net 5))
 (segment (start 226.18 76.67) (end 227.655 78.145) (width 0.4064) (layer "B.Cu") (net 5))
 (segment (start 225.195 97.82) (end 224.58 97.205) (width 0.4064) (layer "B.Cu") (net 5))
 (segment (start 228.24 77.56) (end 229.887584 77.56) (width 0.4064) (layer "B.Cu") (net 5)))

